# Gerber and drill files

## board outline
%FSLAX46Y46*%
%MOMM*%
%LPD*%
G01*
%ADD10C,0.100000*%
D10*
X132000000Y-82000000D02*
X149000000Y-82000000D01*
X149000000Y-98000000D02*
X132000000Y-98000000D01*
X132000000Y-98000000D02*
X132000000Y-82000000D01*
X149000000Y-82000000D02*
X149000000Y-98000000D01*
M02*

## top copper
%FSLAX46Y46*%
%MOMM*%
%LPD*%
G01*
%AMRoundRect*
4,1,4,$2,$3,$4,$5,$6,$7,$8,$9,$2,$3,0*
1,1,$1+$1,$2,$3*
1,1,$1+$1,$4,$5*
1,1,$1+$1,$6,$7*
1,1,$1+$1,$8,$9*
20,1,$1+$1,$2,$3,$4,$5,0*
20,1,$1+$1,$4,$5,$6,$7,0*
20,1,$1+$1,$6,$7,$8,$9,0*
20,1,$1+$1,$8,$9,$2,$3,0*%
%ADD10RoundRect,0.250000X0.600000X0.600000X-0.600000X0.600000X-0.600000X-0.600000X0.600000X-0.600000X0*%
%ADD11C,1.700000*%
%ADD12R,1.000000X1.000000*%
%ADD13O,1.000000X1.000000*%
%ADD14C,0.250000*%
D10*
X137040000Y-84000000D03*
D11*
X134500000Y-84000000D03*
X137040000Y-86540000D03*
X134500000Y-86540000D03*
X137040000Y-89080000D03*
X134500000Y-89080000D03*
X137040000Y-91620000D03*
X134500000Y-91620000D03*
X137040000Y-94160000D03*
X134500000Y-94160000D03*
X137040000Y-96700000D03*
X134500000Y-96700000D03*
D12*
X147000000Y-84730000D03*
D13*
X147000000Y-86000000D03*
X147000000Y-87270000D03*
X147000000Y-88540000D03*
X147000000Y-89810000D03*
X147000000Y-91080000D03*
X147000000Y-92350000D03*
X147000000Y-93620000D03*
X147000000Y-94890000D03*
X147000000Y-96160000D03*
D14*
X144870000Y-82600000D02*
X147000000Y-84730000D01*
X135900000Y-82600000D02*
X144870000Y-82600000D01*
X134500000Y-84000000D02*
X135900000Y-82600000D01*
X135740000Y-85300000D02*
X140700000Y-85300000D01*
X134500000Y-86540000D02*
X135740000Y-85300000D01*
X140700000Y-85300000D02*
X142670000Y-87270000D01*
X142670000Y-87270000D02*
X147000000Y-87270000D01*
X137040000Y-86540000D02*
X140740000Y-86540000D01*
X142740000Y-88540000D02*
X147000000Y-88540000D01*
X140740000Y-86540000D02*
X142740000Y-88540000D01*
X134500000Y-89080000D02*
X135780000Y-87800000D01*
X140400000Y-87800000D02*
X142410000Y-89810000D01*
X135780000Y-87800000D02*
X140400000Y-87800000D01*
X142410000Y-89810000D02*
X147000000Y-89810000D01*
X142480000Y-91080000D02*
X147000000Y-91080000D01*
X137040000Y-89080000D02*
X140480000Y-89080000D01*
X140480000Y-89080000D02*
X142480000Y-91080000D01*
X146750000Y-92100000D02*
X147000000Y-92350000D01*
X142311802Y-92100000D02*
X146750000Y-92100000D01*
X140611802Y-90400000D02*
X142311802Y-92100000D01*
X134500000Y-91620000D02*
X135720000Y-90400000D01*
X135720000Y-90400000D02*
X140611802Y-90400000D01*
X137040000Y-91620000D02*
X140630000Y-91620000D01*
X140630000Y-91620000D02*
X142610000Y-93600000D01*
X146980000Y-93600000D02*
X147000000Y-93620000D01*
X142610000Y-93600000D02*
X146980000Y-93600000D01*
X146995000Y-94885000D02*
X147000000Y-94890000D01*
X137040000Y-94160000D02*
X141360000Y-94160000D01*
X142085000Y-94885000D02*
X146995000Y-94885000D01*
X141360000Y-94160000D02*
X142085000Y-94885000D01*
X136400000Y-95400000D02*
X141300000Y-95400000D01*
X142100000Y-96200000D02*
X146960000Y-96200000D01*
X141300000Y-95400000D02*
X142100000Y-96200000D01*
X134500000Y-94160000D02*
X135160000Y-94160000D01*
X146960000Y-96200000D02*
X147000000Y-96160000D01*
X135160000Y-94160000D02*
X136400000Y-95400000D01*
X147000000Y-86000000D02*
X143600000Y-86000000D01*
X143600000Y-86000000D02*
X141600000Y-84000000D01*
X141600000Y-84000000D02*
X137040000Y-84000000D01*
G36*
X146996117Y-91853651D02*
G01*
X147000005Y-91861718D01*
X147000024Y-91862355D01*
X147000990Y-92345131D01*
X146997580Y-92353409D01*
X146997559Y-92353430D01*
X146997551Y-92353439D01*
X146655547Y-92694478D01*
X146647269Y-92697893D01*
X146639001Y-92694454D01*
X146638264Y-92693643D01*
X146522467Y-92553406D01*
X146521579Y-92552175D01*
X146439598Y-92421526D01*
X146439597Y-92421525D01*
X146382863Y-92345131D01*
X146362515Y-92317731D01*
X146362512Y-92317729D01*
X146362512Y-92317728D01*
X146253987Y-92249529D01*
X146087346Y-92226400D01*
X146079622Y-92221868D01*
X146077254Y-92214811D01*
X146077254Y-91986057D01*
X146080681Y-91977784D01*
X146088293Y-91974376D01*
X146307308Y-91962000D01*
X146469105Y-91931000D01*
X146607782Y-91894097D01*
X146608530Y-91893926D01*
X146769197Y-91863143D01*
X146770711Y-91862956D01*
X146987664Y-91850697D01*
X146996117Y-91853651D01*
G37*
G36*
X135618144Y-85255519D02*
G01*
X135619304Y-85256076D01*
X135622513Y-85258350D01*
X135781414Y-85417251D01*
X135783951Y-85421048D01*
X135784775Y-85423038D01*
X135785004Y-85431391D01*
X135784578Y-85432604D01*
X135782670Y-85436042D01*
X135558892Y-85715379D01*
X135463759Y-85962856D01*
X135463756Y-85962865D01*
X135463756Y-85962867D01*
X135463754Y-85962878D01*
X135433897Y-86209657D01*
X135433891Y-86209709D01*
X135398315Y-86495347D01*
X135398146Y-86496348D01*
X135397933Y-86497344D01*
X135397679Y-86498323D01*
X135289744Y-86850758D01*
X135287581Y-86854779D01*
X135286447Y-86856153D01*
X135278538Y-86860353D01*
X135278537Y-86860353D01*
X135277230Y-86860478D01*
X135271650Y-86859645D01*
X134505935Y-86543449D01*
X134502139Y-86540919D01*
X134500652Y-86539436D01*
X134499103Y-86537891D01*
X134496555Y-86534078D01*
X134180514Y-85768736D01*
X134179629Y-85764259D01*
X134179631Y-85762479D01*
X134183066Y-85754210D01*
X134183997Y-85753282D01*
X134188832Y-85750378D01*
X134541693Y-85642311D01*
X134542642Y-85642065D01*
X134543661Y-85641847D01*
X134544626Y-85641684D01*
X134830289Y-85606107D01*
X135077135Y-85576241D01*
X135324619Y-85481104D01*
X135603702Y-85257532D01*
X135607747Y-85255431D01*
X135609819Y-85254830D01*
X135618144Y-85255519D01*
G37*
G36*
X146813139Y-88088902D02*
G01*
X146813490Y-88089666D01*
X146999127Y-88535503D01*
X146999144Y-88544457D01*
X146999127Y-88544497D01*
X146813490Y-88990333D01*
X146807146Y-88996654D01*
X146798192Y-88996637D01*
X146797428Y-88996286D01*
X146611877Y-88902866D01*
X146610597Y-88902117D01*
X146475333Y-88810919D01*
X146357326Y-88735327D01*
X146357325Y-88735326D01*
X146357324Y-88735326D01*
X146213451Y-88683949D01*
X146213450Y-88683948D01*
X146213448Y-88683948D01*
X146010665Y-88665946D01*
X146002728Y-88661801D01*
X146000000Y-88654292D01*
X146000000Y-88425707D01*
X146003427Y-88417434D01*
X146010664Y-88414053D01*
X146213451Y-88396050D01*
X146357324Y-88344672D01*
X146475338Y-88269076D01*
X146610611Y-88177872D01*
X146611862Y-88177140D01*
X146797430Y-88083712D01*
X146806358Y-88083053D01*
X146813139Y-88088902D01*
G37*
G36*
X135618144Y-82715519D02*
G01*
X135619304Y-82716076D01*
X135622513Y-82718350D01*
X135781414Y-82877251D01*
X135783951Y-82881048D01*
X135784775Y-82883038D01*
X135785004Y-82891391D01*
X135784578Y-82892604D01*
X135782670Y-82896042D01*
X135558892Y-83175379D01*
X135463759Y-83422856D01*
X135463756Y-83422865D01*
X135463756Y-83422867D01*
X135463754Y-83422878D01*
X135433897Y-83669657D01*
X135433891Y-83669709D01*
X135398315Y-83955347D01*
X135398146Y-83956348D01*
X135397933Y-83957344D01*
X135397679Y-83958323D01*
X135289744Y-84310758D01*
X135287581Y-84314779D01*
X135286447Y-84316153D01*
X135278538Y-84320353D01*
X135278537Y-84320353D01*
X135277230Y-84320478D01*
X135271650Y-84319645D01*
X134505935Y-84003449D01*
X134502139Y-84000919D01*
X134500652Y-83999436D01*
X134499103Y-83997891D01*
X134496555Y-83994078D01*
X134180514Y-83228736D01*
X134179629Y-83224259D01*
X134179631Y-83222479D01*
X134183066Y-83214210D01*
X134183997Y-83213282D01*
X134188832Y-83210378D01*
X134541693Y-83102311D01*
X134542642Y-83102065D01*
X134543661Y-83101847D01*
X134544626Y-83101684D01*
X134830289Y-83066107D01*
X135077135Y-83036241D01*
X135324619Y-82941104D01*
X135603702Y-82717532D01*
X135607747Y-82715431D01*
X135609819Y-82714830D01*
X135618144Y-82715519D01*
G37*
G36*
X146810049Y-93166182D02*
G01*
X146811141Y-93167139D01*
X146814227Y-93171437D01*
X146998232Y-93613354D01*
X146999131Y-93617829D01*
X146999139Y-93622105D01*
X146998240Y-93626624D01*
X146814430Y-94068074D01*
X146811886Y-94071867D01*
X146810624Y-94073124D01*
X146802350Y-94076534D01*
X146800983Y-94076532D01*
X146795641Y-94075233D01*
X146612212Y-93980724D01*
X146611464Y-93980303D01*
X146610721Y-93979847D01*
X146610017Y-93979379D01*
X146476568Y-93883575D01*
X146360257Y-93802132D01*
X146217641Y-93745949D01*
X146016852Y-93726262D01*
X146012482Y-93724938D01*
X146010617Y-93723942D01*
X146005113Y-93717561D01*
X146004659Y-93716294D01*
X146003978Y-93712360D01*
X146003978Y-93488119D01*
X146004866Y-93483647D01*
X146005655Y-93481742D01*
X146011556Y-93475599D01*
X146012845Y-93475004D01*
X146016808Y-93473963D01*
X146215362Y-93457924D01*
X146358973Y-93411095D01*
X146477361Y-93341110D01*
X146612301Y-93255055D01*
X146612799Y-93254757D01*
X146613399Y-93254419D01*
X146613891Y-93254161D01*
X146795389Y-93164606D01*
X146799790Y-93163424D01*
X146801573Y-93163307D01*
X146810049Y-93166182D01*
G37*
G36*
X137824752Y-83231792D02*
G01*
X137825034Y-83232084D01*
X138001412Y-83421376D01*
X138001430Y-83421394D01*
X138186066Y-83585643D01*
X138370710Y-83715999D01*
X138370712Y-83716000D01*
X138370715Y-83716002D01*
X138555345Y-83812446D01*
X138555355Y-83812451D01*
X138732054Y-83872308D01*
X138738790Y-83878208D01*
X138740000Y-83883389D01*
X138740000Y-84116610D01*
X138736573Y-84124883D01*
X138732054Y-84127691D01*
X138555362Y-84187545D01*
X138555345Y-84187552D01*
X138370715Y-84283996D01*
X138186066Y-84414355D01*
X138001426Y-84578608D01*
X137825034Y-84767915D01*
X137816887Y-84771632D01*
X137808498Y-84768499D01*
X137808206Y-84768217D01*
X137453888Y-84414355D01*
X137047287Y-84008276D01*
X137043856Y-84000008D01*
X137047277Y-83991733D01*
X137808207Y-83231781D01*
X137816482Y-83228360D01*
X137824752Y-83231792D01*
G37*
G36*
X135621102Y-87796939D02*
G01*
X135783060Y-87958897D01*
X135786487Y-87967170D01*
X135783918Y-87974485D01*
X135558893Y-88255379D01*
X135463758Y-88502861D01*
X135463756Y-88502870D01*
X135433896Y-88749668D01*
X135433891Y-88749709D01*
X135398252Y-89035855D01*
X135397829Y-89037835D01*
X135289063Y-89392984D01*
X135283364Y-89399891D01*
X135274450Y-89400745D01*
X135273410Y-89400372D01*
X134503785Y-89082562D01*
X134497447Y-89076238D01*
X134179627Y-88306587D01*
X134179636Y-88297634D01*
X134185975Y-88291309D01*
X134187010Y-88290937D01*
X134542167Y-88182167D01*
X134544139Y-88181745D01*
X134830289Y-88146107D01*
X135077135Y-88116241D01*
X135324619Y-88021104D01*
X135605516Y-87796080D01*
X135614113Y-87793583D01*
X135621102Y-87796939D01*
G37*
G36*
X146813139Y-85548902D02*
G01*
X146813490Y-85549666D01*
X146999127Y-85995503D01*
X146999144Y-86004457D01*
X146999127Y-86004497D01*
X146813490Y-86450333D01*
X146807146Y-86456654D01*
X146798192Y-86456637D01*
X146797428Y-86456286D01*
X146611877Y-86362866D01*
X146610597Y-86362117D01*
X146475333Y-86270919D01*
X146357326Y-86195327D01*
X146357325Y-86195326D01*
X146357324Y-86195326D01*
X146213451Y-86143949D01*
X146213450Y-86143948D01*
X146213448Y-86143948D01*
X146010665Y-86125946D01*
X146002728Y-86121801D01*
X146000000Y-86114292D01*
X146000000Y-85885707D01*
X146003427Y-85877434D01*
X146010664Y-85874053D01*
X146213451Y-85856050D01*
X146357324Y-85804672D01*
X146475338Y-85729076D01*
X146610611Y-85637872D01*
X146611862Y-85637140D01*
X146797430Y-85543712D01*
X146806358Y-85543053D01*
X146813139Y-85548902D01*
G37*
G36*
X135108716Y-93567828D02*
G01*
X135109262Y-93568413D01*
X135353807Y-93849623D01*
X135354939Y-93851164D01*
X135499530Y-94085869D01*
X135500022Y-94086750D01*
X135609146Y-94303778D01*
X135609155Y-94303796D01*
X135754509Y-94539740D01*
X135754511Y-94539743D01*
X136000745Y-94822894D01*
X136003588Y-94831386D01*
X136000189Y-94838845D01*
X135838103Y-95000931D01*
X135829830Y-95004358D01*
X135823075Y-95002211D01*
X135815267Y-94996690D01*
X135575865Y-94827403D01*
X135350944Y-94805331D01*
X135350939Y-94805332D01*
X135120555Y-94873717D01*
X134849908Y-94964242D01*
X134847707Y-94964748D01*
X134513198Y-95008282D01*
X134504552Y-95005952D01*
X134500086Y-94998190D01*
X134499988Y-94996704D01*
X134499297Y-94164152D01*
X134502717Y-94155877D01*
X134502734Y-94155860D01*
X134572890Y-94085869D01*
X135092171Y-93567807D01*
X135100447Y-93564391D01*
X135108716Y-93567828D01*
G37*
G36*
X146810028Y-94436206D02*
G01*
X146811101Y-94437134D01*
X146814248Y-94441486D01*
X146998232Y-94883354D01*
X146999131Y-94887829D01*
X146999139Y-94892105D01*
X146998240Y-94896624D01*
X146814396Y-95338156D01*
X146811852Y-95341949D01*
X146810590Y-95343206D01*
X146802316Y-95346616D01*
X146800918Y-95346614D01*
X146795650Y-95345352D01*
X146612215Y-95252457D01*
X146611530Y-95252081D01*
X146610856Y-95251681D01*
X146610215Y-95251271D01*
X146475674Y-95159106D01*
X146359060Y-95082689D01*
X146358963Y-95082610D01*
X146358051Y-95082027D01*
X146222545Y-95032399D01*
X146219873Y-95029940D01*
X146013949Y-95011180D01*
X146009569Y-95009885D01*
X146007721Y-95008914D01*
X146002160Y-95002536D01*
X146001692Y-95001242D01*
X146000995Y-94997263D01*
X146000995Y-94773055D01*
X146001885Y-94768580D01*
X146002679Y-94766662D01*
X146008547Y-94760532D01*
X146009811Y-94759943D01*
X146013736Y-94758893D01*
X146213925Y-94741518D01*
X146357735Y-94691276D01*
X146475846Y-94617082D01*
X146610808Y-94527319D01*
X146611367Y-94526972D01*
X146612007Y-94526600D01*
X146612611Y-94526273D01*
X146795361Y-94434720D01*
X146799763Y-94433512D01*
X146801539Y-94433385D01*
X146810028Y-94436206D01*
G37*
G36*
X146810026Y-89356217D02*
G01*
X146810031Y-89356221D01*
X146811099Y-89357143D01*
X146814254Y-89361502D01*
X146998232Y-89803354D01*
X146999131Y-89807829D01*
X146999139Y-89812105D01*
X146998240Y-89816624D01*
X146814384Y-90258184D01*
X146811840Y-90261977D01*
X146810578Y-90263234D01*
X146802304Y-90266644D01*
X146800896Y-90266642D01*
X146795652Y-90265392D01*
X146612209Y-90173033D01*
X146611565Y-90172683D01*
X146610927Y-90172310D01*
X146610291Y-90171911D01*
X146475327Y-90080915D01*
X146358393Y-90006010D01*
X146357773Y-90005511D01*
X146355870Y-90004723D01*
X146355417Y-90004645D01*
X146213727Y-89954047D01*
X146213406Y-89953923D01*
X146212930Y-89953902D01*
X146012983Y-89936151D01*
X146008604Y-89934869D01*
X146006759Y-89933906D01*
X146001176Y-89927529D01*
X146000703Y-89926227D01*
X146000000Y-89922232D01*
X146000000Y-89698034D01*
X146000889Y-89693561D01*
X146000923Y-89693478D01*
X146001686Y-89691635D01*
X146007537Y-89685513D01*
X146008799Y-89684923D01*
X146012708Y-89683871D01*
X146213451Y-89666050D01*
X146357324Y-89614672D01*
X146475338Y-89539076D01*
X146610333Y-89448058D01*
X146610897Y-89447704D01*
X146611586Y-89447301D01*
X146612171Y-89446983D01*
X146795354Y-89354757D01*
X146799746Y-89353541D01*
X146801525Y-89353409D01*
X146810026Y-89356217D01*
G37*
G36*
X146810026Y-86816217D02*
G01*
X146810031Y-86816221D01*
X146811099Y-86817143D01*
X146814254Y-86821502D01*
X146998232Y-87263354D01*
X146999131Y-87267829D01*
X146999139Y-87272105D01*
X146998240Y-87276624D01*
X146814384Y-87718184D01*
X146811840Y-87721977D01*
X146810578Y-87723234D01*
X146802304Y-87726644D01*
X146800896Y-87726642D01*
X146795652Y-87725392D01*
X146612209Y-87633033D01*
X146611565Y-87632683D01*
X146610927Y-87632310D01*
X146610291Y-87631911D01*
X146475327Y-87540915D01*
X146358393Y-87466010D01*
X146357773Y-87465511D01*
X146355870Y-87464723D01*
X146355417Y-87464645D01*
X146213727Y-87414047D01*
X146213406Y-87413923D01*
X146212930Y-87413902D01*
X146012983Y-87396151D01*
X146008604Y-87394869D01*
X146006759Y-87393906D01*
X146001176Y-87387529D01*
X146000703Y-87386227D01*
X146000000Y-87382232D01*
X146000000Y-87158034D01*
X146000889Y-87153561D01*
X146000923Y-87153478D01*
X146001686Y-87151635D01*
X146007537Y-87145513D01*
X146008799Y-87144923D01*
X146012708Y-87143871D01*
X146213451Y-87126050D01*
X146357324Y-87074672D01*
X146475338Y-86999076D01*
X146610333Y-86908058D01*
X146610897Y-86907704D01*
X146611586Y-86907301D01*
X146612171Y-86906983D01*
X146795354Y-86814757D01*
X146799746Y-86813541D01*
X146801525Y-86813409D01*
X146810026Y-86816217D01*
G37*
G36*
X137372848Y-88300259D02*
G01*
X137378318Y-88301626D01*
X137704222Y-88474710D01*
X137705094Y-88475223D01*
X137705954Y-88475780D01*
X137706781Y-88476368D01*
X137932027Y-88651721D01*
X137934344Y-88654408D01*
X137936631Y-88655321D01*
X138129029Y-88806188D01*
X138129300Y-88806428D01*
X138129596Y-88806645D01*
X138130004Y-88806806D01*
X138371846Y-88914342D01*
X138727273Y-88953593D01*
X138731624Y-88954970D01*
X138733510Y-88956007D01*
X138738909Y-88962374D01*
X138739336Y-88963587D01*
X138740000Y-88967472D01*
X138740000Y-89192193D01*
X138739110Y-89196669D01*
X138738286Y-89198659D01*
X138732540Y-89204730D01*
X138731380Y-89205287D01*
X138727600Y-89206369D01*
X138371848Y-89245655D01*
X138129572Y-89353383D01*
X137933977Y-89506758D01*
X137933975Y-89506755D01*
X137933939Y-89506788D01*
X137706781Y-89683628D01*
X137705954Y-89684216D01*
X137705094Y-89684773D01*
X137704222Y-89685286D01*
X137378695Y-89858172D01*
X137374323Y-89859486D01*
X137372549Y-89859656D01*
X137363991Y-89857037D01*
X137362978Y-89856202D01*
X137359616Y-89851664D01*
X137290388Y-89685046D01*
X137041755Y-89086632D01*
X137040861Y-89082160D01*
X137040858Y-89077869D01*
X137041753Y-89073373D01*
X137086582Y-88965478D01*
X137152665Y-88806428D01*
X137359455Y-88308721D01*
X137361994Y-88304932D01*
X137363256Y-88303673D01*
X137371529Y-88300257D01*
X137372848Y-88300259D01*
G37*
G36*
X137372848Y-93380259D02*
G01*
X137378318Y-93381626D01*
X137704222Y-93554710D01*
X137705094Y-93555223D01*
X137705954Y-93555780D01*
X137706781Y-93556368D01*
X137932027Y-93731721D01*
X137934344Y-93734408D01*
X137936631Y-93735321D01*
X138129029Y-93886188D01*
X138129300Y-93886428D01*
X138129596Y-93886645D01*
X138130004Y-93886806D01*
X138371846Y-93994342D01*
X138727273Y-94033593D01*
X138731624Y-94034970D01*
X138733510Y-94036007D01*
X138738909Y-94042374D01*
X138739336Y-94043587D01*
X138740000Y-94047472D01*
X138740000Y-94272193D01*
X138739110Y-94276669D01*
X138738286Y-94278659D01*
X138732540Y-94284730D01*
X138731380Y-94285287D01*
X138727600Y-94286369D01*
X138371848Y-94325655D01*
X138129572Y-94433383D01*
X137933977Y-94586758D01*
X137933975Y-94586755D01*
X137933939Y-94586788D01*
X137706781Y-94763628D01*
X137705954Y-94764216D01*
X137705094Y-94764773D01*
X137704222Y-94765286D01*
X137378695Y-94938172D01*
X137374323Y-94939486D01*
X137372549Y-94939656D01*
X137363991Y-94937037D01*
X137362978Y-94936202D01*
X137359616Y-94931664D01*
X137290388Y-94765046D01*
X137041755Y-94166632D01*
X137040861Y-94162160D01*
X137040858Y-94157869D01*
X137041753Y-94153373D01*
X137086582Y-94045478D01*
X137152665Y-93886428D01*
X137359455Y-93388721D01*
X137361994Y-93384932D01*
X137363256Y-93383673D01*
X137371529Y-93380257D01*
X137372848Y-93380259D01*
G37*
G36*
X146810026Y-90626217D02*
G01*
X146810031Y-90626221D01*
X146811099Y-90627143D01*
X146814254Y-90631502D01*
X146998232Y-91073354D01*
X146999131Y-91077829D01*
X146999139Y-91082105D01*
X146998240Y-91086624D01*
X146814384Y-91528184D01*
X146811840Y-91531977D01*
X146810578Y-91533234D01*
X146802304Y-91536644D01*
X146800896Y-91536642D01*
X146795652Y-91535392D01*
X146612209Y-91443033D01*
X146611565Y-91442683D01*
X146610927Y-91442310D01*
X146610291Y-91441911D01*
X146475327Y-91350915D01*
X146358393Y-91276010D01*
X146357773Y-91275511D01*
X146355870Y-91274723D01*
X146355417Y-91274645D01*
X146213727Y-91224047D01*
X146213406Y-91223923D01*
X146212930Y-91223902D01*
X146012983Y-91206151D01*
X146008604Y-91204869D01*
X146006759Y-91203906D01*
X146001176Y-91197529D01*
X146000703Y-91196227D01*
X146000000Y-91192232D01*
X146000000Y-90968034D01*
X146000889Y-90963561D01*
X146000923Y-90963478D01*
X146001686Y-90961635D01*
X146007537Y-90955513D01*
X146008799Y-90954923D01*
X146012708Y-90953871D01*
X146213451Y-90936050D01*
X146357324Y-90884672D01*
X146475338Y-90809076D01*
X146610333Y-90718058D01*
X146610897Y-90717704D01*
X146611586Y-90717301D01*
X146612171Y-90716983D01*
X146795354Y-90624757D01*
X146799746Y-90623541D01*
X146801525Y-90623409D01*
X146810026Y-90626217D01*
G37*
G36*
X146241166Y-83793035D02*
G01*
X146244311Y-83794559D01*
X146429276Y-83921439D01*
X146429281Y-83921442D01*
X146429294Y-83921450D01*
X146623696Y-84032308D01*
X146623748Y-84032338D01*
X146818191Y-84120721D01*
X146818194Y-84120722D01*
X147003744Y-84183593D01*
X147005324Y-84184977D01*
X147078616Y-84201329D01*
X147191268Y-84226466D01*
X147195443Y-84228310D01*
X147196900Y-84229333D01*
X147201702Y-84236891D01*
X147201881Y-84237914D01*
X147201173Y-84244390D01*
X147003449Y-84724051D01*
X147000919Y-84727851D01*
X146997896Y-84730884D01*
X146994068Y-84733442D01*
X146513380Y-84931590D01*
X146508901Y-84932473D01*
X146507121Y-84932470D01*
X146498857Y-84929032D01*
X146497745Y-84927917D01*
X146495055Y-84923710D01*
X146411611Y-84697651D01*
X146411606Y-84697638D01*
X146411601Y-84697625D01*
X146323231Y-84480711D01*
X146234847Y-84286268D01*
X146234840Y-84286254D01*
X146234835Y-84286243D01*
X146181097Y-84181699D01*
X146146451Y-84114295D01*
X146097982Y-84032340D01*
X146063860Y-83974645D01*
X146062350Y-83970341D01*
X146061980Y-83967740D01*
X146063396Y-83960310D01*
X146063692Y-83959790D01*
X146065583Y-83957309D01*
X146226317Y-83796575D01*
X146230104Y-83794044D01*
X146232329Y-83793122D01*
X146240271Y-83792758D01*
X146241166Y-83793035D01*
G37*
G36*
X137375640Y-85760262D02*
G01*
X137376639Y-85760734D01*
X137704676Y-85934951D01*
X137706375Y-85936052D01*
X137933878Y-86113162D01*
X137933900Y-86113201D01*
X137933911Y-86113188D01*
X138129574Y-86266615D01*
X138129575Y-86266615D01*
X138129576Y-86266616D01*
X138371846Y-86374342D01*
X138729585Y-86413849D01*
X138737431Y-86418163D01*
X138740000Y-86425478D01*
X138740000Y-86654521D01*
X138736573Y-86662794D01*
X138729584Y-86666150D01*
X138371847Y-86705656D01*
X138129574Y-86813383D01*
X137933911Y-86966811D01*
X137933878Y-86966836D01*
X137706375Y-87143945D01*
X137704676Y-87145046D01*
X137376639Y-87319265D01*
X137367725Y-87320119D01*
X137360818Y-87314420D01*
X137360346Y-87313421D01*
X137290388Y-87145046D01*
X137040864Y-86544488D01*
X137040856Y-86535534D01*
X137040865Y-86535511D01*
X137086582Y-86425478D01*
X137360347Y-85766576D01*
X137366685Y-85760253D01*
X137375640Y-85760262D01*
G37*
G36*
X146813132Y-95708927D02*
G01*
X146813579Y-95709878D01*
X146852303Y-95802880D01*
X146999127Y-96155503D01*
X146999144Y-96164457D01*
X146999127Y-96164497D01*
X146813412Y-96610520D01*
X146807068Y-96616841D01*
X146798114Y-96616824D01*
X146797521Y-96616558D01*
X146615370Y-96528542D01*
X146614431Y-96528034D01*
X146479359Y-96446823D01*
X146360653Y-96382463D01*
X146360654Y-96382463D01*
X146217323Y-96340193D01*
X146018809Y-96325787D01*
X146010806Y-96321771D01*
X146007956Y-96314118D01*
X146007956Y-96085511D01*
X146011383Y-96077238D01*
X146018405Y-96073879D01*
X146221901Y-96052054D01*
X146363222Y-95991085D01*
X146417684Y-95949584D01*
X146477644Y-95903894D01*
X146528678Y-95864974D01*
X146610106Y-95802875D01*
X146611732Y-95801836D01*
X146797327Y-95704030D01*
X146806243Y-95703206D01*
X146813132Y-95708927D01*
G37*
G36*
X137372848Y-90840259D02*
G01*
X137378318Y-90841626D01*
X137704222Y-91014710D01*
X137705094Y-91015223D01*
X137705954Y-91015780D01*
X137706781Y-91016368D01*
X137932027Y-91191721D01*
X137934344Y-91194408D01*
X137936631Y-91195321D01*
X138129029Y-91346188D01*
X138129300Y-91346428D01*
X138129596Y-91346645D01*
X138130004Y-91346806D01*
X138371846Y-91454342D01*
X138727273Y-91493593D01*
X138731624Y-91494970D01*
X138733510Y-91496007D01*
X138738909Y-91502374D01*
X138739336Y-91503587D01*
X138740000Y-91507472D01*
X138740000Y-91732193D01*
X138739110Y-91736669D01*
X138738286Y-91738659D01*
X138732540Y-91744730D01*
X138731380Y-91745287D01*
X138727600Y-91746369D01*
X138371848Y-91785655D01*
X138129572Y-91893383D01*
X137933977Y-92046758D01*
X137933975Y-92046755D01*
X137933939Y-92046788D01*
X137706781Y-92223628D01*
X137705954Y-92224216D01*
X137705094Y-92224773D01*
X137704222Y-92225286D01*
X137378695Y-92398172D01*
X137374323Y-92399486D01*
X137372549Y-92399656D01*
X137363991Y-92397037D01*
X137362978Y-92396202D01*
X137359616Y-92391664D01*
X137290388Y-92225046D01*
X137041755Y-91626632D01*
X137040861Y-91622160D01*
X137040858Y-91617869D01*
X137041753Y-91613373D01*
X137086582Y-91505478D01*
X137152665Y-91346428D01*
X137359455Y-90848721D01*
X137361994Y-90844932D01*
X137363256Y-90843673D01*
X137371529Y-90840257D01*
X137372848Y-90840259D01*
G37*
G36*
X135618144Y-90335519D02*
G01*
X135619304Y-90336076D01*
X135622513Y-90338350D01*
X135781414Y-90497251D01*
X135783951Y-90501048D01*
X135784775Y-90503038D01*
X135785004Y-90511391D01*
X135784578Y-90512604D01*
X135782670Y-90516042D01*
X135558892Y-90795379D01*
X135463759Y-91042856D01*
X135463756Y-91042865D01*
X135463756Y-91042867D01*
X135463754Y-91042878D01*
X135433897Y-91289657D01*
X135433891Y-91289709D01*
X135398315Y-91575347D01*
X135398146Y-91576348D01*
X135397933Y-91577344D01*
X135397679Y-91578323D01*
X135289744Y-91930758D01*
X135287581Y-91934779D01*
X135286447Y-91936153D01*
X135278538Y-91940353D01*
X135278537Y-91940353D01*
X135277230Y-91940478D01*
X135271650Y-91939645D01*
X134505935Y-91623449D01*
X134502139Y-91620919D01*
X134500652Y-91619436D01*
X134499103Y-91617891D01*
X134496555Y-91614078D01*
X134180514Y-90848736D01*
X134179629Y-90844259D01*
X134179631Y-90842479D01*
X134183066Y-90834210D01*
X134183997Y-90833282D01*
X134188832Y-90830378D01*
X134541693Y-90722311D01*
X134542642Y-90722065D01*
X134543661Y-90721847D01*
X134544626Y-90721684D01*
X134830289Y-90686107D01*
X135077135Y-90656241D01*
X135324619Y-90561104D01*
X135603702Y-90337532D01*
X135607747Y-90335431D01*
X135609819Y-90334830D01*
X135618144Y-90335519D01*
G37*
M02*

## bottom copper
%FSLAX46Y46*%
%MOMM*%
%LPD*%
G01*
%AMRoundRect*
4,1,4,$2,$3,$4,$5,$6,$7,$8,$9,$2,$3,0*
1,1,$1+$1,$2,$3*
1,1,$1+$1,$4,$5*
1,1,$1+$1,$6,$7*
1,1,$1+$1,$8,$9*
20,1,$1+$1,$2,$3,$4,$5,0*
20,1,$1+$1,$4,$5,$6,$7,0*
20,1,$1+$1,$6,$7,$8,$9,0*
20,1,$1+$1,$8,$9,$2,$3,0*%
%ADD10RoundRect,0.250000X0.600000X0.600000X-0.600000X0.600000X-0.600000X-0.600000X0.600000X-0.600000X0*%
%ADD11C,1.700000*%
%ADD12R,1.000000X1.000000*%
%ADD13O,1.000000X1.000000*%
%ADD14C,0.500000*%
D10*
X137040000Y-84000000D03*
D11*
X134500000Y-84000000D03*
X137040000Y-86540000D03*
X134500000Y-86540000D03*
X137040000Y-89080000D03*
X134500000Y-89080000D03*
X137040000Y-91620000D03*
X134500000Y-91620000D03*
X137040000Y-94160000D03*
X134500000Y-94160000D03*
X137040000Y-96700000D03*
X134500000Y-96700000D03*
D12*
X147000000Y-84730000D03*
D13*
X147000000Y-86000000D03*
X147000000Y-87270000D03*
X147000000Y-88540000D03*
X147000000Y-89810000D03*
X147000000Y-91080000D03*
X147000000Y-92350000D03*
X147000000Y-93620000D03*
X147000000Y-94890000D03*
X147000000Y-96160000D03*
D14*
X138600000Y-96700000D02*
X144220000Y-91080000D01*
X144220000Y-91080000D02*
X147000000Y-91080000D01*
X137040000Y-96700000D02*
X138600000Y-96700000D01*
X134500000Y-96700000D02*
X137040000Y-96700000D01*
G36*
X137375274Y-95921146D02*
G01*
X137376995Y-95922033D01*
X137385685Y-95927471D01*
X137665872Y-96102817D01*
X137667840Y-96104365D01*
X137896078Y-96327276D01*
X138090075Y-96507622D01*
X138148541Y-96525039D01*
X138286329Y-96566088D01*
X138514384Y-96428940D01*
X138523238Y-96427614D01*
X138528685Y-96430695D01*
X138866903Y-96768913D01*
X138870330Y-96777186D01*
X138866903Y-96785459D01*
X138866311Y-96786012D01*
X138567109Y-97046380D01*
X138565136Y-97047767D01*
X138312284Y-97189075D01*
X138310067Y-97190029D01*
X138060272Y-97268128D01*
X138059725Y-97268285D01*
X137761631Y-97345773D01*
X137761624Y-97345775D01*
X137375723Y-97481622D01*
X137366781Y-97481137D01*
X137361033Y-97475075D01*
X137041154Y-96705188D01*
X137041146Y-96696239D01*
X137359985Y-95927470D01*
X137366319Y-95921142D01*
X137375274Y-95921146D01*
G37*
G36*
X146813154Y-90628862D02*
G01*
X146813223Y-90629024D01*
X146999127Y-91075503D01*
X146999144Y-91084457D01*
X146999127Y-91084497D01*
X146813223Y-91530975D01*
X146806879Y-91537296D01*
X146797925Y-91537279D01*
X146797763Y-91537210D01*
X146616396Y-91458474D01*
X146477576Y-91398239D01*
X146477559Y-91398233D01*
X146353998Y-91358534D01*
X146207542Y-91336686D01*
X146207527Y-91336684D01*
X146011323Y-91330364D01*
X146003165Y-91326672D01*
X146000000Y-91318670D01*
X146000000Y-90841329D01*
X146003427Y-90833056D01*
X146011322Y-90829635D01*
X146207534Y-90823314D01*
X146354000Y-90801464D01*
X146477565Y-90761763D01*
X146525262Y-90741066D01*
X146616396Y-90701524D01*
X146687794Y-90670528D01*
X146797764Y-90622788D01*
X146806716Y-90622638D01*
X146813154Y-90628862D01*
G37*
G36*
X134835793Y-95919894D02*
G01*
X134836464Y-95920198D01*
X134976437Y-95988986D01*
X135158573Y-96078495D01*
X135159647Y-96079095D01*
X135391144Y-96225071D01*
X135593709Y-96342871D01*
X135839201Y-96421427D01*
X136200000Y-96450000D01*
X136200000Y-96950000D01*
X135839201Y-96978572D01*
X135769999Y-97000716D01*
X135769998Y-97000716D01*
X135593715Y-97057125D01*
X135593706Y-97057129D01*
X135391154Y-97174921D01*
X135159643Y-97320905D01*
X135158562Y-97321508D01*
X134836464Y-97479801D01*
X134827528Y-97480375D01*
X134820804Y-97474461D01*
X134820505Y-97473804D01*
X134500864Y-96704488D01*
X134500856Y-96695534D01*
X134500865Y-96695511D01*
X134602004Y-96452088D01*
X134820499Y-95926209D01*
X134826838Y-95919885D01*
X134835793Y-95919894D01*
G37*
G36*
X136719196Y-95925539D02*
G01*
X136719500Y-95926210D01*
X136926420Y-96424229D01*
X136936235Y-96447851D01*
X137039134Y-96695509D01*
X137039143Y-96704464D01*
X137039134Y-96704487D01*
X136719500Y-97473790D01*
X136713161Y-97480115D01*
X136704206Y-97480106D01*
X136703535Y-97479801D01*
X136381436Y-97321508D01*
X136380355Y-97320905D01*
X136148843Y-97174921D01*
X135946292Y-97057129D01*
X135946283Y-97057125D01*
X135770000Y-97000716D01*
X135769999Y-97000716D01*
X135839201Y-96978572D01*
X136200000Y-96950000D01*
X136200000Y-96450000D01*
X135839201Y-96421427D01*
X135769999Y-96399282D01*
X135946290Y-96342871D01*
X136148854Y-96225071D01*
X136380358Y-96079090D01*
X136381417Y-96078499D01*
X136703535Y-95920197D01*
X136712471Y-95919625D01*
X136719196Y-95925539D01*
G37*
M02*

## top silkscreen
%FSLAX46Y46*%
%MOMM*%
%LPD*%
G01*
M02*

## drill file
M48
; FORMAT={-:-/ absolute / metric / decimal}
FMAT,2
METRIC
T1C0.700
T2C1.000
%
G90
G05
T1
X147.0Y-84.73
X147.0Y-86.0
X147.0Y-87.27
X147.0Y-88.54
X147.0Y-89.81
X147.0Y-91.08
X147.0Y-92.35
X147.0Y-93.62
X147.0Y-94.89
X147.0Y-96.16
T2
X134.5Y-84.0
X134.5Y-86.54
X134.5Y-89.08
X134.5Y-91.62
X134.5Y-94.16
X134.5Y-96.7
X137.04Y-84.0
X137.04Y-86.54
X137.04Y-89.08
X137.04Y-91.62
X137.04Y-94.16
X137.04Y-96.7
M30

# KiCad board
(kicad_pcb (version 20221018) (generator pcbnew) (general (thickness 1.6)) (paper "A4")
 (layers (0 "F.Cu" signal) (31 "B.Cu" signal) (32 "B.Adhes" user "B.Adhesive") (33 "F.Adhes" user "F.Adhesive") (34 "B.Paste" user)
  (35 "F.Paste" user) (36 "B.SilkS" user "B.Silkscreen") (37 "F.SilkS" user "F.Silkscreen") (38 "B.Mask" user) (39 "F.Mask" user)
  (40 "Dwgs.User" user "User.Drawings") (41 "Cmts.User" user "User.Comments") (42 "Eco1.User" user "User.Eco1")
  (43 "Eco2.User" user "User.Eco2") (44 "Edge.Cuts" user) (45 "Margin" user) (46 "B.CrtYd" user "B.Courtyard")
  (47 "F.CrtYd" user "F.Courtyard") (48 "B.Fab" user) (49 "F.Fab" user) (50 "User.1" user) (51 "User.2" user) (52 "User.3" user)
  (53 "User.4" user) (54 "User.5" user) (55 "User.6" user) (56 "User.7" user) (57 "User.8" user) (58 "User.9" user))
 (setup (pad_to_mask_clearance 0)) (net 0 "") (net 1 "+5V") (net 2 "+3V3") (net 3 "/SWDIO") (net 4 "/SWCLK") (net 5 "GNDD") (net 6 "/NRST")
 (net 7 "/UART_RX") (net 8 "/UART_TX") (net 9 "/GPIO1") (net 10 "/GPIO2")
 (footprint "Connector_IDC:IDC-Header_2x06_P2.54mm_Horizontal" (layer "B.Cu") (at 137.04 84 180)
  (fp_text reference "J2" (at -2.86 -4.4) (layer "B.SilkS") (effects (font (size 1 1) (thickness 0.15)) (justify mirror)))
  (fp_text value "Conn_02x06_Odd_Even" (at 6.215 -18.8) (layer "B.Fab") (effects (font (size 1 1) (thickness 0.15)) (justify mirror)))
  (pad "1" thru_hole roundrect (at 0 0 180) (size 1.7 1.7) (drill 1) (layers "*.Cu" "*.Mask") (roundrect_rratio 0.147059) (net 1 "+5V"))
  (pad "2" thru_hole circle (at 2.54 0 180) (size 1.7 1.7) (drill 1) (layers "*.Cu" "*.Mask") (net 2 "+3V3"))
  (pad "3" thru_hole circle (at 0 -2.54 180) (size 1.7 1.7) (drill 1) (layers "*.Cu" "*.Mask") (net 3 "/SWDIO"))
  (pad "4" thru_hole circle (at 2.54 -2.54 180) (size 1.7 1.7) (drill 1) (layers "*.Cu" "*.Mask") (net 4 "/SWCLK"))
  (pad "5" thru_hole circle (at 0 -5.08 180) (size 1.7 1.7) (drill 1) (layers "*.Cu" "*.Mask") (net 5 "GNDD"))
  (pad "6" thru_hole circle (at 2.54 -5.08 180) (size 1.7 1.7) (drill 1) (layers "*.Cu" "*.Mask") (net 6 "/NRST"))
  (pad "7" thru_hole circle (at 0 -7.62 180) (size 1.7 1.7) (drill 1) (layers "*.Cu" "*.Mask") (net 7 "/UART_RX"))
  (pad "8" thru_hole circle (at 2.54 -7.62 180) (size 1.7 1.7) (drill 1) (layers "*.Cu" "*.Mask") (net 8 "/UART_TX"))
  (pad "9" thru_hole circle (at 0 -10.16 180) (size 1.7 1.7) (drill 1) (layers "*.Cu" "*.Mask") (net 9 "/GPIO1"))
  (pad "10" thru_hole circle (at 2.54 -10.16 180) (size 1.7 1.7) (drill 1) (layers "*.Cu" "*.Mask") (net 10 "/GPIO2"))
  (pad "11" thru_hole circle (at 0 -12.7 180) (size 1.7 1.7) (drill 1) (layers "*.Cu" "*.Mask") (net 5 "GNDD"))
  (pad "12" thru_hole circle (at 2.54 -12.7 180) (size 1.7 1.7) (drill 1) (layers "*.Cu" "*.Mask") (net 5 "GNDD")))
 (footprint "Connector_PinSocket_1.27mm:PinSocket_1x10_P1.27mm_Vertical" (layer "B.Cu") (at 147 84.73 180)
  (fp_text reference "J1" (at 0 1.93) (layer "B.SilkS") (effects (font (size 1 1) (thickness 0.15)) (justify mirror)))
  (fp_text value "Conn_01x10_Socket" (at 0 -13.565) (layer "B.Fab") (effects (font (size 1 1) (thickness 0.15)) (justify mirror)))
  (pad "1" thru_hole rect (at 0 0 180) (size 1 1) (drill 0.7) (layers "*.Cu" "*.Mask") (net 2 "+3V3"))
  (pad "2" thru_hole oval (at 0 -1.27 180) (size 1 1) (drill 0.7) (layers "*.Cu" "*.Mask") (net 1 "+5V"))
  (pad "3" thru_hole oval (at 0 -2.54 180) (size 1 1) (drill 0.7) (layers "*.Cu" "*.Mask") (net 4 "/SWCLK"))
  (pad "4" thru_hole oval (at 0 -3.81 180) (size 1 1) (drill 0.7) (layers "*.Cu" "*.Mask") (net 3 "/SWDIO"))
  (pad "5" thru_hole oval (at 0 -5.08 180) (size 1 1) (drill 0.7) (layers "*.Cu" "*.Mask") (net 6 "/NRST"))
  (pad "6" thru_hole oval (at 0 -6.35 180) (size 1 1) (drill 0.7) (layers "*.Cu" "*.Mask") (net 5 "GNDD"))
  (pad "7" thru_hole oval (at 0 -7.62 180) (size 1 1) (drill 0.7) (layers "*.Cu" "*.Mask") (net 8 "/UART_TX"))
  (pad "8" thru_hole oval (at 0 -8.89 180) (size 1 1) (drill 0.7) (layers "*.Cu" "*.Mask") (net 7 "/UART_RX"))
  (pad "9" thru_hole oval (at 0 -10.16 180) (size 1 1) (drill 0.7) (layers "*.Cu" "*.Mask") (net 9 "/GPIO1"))
  (pad "10" thru_hole oval (at 0 -11.43 180) (size 1 1) (drill 0.7) (layers "*.Cu" "*.Mask") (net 10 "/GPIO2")))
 (gr_line (start 132 82) (end 149 82) (stroke (width 0.1) (type default)) (layer "Edge.Cuts"))
 (gr_line (start 149 98) (end 132 98) (stroke (width 0.1) (type default)) (layer "Edge.Cuts"))
 (gr_line (start 132 98) (end 132 82) (stroke (width 0.1) (type default)) (layer "Edge.Cuts"))
 (gr_line (start 149 82) (end 149 98) (stroke (width 0.1) (type default)) (layer "Edge.Cuts"))
 (segment (start 144.87 82.6) (end 147 84.73) (width 0.25) (layer "F.Cu") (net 2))
 (segment (start 135.9 82.6) (end 144.87 82.6) (width 0.25) (layer "F.Cu") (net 2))
 (segment (start 134.5 84) (end 135.9 82.6) (width 0.25) (layer "F.Cu") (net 2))
 (segment (start 135.74 85.3) (end 140.7 85.3) (width 0.25) (layer "F.Cu") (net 4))
 (segment (start 134.5 86.54) (end 135.74 85.3) (width 0.25) (layer "F.Cu") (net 4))
 (segment (start 140.7 85.3) (end 142.67 87.27) (width 0.25) (layer "F.Cu") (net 4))
 (segment (start 142.67 87.27) (end 147 87.27) (width 0.25) (layer "F.Cu") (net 4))
 (segment (start 137.04 86.54) (end 140.74 86.54) (width 0.25) (layer "F.Cu") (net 3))
 (segment (start 142.74 88.54) (end 147 88.54) (width 0.25) (layer "F.Cu") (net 3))
 (segment (start 140.74 86.54) (end 142.74 88.54) (width 0.25) (layer "F.Cu") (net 3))
 (segment (start 134.5 89.08) (end 135.78 87.8) (width 0.25) (layer "F.Cu") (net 6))
 (segment (start 140.4 87.8) (end 142.41 89.81) (width 0.25) (layer "F.Cu") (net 6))
 (segment (start 135.78 87.8) (end 140.4 87.8) (width 0.25) (layer "F.Cu") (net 6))
 (segment (start 142.41 89.81) (end 147 89.81) (width 0.25) (layer "F.Cu") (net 6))
 (segment (start 142.48 91.08) (end 147 91.08) (width 0.25) (layer "F.Cu") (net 5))
 (segment (start 137.04 89.08) (end 140.48 89.08) (width 0.25) (layer "F.Cu") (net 5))
 (segment (start 140.48 89.08) (end 142.48 91.08) (width 0.25) (layer "F.Cu") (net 5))
 (segment (start 138.6 96.7) (end 144.22 91.08) (width 0.5) (layer "B.Cu") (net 5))
 (segment (start 144.22 91.08) (end 147 91.08) (width 0.5) (layer "B.Cu") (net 5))
 (segment (start 137.04 96.7) (end 138.6 96.7) (width 0.5) (layer "B.Cu") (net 5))
 (segment (start 134.5 96.7) (end 137.04 96.7) (width 0.5) (layer "B.Cu") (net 5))
 (segment (start 146.75 92.1) (end 147 92.35) (width 0.25) (layer "F.Cu") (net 8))
 (segment (start 142.311802 92.1) (end 146.75 92.1) (width 0.25) (layer "F.Cu") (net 8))
 (segment (start 140.611802 90.4) (end 142.311802 92.1) (width 0.25) (layer "F.Cu") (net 8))
 (segment (start 134.5 91.62) (end 135.72 90.4) (width 0.25) (layer "F.Cu") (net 8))
 (segment (start 135.72 90.4) (end 140.611802 90.4) (width 0.25) (layer "F.Cu") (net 8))
 (segment (start 137.04 91.62) (end 140.63 91.62) (width 0.25) (layer "F.Cu") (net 7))
 (segment (start 140.63 91.62) (end 142.61 93.6) (width 0.25) (layer "F.Cu") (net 7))
 (segment (start 146.98 93.6) (end 147 93.62) (width 0.25) (layer "F.Cu") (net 7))
 (segment (start 142.61 93.6) (end 146.98 93.6) (width 0.25) (layer "F.Cu") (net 7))
 (segment (start 146.995 94.885) (end 147 94.89) (width 0.25) (layer "F.Cu") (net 9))
 (segment (start 137.04 94.16) (end 141.36 94.16) (width 0.25) (layer "F.Cu") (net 9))
 (segment (start 142.085 94.885) (end 146.995 94.885) (width 0.25) (layer "F.Cu") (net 9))
 (segment (start 141.36 94.16) (end 142.085 94.885) (width 0.25) (layer "F.Cu") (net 9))
 (segment (start 136.4 95.4) (end 141.3 95.4) (width 0.25) (layer "F.Cu") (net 10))
 (segment (start 142.1 96.2) (end 146.96 96.2) (width 0.25) (layer "F.Cu") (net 10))
 (segment (start 141.3 95.4) (end 142.1 96.2) (width 0.25) (layer "F.Cu") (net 10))
 (segment (start 134.5 94.16) (end 135.16 94.16) (width 0.25) (layer "F.Cu") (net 10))
 (segment (start 146.96 96.2) (end 147 96.16) (width 0.25) (layer "F.Cu") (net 10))
 (segment (start 135.16 94.16) (end 136.4 95.4) (width 0.25) (layer "F.Cu") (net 10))
 (segment (start 147 86) (end 143.6 86) (width 0.25) (layer "F.Cu") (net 1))
 (segment (start 143.6 86) (end 141.6 84) (width 0.25) (layer "F.Cu") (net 1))
 (segment (start 141.6 84) (end 137.04 84) (width 0.25) (layer "F.Cu") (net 1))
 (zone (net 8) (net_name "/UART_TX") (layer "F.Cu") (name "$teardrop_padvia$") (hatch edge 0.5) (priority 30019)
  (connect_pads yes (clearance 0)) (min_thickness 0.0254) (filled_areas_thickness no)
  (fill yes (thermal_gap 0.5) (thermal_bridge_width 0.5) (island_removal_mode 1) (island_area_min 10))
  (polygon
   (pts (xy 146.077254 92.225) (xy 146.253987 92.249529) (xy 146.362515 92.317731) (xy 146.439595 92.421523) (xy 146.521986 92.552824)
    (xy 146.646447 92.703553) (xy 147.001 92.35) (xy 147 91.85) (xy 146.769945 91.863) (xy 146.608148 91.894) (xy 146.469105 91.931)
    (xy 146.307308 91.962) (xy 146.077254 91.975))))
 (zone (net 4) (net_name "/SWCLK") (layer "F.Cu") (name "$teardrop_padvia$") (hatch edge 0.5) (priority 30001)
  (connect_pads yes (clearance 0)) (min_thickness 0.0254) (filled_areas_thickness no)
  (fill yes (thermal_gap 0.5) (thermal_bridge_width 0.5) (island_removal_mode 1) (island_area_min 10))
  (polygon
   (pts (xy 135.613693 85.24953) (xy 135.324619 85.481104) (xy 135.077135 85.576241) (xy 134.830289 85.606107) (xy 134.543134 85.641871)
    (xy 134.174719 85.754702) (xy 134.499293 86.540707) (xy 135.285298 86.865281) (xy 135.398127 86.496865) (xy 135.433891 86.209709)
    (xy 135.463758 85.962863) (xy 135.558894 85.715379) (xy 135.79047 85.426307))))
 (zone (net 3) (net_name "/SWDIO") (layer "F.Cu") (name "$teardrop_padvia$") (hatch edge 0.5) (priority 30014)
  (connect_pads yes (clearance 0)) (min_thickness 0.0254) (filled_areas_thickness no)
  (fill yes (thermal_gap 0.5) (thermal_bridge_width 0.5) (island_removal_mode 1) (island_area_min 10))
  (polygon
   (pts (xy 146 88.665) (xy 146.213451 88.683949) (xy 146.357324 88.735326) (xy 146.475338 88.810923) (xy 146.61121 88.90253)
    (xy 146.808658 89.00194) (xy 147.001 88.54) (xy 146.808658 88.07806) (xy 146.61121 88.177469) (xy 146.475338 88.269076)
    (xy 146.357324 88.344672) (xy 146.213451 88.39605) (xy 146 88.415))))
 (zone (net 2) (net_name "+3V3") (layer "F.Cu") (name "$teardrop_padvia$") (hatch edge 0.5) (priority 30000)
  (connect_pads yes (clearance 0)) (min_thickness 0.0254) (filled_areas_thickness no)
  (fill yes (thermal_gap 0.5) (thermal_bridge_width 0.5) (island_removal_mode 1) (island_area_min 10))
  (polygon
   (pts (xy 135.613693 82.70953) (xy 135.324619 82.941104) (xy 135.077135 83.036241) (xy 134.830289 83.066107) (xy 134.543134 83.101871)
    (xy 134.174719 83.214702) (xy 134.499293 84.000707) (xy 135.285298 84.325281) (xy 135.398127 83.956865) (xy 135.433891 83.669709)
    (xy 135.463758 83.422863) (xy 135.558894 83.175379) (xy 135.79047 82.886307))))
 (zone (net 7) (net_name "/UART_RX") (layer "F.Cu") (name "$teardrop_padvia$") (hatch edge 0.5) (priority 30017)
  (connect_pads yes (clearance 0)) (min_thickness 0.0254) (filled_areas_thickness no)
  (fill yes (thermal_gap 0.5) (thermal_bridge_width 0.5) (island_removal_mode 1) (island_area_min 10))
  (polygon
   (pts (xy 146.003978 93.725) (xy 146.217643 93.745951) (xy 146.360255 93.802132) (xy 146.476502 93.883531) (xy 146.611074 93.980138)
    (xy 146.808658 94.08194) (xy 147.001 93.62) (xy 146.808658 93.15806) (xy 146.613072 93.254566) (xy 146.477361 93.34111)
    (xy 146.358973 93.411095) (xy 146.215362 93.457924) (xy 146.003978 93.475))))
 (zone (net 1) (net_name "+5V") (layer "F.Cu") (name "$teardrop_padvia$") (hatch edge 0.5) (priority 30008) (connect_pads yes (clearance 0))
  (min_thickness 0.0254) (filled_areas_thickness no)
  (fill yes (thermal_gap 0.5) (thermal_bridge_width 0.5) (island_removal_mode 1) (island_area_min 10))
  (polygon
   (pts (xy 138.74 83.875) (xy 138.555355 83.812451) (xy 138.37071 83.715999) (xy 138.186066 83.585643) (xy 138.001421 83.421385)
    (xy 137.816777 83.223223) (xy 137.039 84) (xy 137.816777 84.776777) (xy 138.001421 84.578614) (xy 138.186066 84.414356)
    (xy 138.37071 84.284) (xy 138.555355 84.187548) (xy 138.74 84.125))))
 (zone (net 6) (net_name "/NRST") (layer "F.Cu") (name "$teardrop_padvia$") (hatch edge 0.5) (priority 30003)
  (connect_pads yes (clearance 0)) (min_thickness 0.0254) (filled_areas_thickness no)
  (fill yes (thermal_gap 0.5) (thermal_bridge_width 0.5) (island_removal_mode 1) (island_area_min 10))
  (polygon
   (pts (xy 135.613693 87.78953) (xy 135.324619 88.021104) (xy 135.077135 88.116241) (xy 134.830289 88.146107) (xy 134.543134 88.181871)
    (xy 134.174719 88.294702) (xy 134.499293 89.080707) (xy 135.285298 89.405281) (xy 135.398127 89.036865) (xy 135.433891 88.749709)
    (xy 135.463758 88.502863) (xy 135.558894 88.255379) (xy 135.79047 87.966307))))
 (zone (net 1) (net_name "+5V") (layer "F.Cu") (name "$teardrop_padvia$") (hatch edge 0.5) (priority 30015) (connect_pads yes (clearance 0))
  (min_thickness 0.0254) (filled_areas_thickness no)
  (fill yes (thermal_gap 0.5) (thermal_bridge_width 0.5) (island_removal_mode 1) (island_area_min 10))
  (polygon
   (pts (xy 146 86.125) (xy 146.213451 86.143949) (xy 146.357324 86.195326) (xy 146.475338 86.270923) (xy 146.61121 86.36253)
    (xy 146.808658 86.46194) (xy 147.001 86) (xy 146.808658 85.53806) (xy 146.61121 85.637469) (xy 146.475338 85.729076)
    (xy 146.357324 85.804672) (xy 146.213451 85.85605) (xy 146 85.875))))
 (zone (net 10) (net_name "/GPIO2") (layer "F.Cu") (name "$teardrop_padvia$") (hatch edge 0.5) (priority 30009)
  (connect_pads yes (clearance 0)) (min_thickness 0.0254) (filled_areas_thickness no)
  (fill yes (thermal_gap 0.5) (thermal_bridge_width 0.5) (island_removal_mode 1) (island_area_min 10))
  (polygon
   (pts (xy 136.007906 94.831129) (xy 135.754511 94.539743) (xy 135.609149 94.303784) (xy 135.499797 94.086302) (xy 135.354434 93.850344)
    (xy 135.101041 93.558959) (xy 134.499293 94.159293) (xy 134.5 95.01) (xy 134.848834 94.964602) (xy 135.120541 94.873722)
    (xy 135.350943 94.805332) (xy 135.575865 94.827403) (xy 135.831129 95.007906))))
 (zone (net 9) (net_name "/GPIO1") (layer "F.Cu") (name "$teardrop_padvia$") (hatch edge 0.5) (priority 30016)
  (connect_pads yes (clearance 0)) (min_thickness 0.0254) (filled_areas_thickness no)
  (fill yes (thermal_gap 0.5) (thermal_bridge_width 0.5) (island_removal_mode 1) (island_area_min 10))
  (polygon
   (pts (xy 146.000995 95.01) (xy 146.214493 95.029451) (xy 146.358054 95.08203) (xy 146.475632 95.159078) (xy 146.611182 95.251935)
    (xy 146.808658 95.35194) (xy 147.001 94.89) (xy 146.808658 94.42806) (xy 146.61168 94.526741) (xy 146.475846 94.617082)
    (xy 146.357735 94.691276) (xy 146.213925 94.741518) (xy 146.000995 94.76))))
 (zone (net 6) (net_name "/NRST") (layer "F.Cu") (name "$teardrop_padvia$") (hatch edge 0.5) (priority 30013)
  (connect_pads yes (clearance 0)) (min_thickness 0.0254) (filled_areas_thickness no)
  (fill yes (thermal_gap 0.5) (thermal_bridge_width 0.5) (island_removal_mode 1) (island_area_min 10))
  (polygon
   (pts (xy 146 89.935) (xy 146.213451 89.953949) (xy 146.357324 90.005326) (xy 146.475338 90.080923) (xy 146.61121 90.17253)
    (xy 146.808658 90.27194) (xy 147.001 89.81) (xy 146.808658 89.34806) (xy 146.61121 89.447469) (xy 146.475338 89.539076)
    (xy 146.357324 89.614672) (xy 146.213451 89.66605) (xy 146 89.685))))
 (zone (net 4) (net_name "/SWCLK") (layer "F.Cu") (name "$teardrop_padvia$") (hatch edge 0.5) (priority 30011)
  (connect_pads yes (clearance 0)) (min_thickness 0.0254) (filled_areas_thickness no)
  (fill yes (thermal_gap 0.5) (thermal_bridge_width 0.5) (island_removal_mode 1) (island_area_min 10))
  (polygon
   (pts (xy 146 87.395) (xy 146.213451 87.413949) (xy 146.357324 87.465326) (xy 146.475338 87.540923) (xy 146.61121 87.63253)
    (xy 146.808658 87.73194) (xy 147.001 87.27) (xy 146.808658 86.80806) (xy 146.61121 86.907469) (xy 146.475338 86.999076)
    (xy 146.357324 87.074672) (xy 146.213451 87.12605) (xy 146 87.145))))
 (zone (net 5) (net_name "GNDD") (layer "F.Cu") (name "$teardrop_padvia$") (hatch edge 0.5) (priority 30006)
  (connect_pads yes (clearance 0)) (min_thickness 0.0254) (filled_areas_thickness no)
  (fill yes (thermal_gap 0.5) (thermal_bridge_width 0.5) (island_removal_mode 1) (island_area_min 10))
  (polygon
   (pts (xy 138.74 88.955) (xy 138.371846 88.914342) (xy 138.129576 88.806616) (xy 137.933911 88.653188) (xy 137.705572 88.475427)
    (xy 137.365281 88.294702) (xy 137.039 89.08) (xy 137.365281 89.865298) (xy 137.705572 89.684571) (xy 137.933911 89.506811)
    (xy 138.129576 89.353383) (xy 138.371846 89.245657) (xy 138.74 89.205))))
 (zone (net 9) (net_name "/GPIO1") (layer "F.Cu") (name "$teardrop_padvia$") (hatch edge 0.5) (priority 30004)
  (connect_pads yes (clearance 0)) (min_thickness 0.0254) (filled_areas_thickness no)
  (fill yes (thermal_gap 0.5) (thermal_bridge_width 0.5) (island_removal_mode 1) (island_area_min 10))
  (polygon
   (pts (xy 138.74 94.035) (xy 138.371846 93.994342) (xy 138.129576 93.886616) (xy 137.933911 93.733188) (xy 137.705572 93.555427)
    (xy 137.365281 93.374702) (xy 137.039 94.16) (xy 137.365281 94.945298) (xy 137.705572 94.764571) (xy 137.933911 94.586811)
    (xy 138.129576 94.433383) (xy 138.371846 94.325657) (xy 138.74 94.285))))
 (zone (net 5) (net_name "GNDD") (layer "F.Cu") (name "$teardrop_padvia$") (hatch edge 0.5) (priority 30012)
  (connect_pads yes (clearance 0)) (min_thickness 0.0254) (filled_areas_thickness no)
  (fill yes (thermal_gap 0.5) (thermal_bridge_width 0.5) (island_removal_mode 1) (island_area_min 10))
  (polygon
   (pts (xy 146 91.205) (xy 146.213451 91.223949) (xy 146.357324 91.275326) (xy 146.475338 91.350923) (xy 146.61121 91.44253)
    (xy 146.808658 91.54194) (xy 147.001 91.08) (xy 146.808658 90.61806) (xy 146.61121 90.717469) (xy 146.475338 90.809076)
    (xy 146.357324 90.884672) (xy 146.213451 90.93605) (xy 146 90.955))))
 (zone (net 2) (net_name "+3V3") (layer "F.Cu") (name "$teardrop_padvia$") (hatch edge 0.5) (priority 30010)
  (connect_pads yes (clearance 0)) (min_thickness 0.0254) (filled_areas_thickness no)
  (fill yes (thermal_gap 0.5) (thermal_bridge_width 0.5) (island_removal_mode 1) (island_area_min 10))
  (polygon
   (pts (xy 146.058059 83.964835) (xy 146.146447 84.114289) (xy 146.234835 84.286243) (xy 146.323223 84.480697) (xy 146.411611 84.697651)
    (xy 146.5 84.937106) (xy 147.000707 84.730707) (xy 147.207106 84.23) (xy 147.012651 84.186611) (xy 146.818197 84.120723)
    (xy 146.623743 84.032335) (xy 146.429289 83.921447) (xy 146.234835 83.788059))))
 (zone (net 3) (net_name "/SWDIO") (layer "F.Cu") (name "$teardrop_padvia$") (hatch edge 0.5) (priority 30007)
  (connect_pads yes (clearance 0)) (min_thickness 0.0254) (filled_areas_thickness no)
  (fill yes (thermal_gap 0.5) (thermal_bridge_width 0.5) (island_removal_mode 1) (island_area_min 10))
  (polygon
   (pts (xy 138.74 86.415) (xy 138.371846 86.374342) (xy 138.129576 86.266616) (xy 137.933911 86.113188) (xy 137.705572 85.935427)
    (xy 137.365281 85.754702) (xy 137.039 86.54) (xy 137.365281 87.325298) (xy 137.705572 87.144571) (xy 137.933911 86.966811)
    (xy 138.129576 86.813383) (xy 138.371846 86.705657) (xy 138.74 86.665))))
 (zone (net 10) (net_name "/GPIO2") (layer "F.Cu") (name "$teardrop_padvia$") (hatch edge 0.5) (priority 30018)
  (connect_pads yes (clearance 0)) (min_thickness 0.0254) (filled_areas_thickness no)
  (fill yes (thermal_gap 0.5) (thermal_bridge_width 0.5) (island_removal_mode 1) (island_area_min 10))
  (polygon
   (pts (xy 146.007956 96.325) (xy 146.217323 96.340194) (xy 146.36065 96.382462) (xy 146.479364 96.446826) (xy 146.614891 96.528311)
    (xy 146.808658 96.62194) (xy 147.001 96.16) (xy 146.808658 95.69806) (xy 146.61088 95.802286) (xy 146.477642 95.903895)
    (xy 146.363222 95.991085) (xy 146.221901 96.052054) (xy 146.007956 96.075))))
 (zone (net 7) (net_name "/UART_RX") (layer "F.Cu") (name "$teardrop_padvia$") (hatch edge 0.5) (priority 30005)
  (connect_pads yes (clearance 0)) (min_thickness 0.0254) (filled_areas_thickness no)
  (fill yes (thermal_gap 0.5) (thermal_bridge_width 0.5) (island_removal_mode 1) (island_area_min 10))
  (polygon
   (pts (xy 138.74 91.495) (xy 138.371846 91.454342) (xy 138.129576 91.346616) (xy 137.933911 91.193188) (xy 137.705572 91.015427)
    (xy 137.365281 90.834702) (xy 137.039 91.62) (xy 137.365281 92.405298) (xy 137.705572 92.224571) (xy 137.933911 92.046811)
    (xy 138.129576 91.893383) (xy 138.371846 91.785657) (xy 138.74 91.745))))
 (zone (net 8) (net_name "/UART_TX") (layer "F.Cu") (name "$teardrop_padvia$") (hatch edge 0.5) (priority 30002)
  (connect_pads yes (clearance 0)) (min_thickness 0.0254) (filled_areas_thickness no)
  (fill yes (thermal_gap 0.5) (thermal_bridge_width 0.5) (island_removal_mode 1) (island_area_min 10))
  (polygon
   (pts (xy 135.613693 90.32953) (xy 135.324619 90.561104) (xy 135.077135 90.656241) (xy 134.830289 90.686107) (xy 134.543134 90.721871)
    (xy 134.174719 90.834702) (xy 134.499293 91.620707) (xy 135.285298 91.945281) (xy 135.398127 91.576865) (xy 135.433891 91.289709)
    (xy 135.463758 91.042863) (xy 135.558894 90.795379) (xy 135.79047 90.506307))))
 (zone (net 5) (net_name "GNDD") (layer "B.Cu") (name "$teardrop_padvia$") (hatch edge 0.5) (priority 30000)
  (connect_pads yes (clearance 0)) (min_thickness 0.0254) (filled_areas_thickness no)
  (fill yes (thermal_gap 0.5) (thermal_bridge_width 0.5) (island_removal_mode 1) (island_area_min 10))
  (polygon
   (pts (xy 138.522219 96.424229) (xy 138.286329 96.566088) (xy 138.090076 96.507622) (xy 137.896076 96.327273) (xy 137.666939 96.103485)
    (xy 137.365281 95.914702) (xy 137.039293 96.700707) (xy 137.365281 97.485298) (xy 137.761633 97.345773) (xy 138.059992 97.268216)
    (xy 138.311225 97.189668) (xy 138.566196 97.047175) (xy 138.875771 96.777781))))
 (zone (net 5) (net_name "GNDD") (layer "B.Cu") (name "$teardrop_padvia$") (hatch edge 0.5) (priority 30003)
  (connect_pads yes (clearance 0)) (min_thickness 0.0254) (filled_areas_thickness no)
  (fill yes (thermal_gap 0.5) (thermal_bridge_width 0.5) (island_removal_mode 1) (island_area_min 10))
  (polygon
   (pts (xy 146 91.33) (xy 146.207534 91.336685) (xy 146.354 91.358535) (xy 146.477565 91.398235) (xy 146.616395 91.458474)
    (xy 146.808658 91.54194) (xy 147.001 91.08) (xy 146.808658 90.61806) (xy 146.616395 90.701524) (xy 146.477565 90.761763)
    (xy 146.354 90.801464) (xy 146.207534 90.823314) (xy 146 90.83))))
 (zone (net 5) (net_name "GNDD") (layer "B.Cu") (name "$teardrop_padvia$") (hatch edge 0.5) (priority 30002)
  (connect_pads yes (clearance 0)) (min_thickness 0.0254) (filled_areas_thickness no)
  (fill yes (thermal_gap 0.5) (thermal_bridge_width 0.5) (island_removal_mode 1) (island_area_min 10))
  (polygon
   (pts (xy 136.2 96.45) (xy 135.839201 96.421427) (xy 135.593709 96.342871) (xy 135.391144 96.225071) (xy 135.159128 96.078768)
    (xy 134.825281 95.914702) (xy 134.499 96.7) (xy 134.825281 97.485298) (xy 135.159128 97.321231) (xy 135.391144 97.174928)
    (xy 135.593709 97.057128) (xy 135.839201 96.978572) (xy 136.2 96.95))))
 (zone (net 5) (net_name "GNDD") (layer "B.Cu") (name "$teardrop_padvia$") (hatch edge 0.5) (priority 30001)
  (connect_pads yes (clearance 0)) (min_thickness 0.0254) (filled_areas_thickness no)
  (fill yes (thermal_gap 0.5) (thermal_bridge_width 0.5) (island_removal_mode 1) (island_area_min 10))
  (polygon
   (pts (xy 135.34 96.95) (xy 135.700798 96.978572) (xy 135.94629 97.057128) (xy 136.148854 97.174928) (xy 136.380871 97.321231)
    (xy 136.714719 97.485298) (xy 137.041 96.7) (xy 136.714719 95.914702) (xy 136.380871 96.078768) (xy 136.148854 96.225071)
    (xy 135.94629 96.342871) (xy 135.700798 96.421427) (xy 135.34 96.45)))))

